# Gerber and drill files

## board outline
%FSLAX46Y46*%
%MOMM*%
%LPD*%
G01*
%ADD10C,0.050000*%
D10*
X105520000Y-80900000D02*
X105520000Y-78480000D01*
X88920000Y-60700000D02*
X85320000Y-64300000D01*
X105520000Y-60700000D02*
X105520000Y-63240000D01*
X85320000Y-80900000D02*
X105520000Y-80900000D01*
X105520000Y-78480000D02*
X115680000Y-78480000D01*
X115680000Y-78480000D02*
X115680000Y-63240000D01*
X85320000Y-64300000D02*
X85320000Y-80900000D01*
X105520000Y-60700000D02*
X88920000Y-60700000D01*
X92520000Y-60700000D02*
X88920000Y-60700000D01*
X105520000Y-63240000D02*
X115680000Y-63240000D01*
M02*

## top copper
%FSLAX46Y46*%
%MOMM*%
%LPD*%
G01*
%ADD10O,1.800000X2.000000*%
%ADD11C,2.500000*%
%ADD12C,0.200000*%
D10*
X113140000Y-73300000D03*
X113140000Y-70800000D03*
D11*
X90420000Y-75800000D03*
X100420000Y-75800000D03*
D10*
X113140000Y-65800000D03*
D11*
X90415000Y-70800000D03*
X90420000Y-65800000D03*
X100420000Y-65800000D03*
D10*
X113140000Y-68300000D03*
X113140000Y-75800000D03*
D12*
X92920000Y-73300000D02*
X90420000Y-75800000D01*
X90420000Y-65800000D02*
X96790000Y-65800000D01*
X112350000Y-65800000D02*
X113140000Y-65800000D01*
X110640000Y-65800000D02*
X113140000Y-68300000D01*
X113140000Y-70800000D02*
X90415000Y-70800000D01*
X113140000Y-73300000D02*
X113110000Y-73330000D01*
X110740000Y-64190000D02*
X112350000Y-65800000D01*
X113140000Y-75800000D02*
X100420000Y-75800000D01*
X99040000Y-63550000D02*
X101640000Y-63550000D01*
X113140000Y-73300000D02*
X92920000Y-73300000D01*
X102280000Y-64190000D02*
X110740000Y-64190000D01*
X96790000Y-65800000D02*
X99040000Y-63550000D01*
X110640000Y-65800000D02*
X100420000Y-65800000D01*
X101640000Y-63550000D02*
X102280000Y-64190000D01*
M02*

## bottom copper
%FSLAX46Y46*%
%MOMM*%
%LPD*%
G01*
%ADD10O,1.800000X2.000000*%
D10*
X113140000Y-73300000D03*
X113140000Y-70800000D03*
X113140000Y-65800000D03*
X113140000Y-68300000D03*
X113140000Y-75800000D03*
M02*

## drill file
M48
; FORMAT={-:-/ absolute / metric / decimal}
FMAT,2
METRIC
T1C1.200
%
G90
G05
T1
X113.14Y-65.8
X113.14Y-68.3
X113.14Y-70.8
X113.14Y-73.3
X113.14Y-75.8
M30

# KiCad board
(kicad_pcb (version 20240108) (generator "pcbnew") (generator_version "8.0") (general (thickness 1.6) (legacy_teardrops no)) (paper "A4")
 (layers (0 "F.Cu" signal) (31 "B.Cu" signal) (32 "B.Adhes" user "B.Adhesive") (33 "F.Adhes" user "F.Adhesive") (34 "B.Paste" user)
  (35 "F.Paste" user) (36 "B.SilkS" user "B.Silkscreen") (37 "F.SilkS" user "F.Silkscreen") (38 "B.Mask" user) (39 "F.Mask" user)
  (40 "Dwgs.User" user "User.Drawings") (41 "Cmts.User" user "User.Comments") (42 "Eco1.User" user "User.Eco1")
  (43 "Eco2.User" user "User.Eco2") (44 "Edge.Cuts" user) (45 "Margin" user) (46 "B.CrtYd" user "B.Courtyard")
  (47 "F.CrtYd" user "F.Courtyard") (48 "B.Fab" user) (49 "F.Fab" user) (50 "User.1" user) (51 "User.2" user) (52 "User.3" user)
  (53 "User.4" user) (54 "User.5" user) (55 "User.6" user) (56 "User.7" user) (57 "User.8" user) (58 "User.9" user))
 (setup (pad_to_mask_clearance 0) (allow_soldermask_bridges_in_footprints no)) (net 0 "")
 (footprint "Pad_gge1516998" (layer "F.Cu") (at 113.14 73.3 180)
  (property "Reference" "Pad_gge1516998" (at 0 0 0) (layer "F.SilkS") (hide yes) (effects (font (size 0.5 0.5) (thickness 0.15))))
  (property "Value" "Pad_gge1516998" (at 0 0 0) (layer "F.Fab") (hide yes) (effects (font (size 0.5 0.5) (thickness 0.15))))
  (pad "2" thru_hole oval (at 0 0 180) (size 1.8 2) (drill 1.2) (layers "*.Cu" "*.Mask") (remove_unused_layers no)
   (solder_mask_margin 0.0508) (thermal_bridge_angle 0)))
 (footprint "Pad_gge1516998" (layer "F.Cu") (at 113.14 70.8 180)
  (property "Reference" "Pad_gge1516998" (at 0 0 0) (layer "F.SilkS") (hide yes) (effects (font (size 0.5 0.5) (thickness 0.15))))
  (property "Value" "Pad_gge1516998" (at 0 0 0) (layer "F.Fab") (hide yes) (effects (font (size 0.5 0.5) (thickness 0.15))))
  (pad "2" thru_hole oval (at 0 0 180) (size 1.8 2) (drill 1.2) (layers "*.Cu" "*.Mask") (remove_unused_layers no)
   (solder_mask_margin 0.0508) (thermal_bridge_angle 0)))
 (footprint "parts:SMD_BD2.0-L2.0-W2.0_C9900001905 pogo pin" (layer "F.Cu") (at 90.42 75.8)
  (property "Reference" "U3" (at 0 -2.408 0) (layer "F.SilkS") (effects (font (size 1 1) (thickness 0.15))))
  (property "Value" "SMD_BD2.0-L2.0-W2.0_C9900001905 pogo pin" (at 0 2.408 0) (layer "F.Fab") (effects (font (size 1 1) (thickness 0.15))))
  (pad "1" smd circle (at 0 0) (size 2.5 2.5) (layers "F.Cu" "F.Paste" "F.Mask") (thermal_bridge_angle 90)))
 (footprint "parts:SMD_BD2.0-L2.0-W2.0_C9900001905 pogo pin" (layer "F.Cu") (at 100.42 75.8)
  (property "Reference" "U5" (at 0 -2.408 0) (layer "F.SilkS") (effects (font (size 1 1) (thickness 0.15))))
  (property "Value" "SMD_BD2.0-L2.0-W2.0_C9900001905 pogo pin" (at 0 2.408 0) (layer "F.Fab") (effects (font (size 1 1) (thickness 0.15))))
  (pad "1" smd circle (at 0 0) (size 2.5 2.5) (layers "F.Cu" "F.Paste" "F.Mask") (thermal_bridge_angle 90)))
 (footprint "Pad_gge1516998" (layer "F.Cu") (at 113.14 65.8 180)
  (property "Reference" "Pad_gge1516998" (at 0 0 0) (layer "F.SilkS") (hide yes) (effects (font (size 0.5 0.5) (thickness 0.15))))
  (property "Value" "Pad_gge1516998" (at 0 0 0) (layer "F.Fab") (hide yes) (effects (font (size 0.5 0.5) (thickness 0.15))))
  (pad "2" thru_hole oval (at 0 0 180) (size 1.8 2) (drill 1.2) (layers "*.Cu" "*.Mask") (remove_unused_layers no)
   (solder_mask_margin 0.0508) (thermal_bridge_angle 0)))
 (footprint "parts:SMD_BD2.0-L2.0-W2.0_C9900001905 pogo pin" (layer "F.Cu") (at 90.415 70.8)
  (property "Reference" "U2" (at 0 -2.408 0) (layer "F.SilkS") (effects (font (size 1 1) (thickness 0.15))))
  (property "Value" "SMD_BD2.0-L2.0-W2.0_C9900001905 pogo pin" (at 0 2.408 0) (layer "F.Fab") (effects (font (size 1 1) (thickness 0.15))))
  (pad "1" smd circle (at 0 0) (size 2.5 2.5) (layers "F.Cu" "F.Paste" "F.Mask") (thermal_bridge_angle 90)))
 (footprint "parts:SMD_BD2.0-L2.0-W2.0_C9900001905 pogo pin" (layer "F.Cu") (at 90.42 65.8)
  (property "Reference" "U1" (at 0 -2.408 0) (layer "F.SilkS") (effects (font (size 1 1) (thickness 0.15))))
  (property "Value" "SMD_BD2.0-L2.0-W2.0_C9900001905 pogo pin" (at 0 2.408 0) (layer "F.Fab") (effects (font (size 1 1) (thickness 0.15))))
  (pad "1" smd circle (at 0 0) (size 2.5 2.5) (layers "F.Cu" "F.Paste" "F.Mask") (thermal_bridge_angle 90)))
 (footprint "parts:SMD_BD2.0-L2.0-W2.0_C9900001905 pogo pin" (layer "F.Cu") (at 100.42 65.8)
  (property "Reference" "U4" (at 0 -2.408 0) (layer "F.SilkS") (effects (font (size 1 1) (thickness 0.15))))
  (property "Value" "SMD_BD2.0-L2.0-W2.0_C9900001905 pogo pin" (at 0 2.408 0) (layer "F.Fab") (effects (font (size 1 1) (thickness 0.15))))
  (pad "1" smd circle (at 0 0) (size 2.5 2.5) (layers "F.Cu" "F.Paste" "F.Mask") (thermal_bridge_angle 90)))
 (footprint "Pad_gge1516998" (layer "F.Cu") (at 113.14 68.3 180)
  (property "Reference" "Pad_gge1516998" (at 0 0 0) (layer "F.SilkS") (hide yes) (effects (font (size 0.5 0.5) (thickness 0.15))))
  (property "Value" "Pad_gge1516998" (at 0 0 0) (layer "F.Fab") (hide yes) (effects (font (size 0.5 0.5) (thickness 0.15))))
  (pad "2" thru_hole oval (at 0 0 180) (size 1.8 2) (drill 1.2) (layers "*.Cu" "*.Mask") (remove_unused_layers no)
   (solder_mask_margin 0.0508) (thermal_bridge_angle 0)))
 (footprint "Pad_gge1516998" (layer "F.Cu") (at 113.14 75.8 180)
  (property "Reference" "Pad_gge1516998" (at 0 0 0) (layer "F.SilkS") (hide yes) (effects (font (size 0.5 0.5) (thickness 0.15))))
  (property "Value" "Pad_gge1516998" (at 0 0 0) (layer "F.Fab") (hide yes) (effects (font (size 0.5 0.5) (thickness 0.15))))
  (pad "2" thru_hole oval (at 0 0 180) (size 1.8 2) (drill 1.2) (layers "*.Cu" "*.Mask") (remove_unused_layers no)
   (solder_mask_margin 0.0508) (thermal_bridge_angle 0)))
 (gr_line (start 105.52 80.9) (end 105.52 78.48) (stroke (width 0.05) (type default)) (layer "Edge.Cuts"))
 (gr_line (start 88.92 60.7) (end 85.32 64.3) (stroke (width 0.05) (type default)) (layer "Edge.Cuts"))
 (gr_line (start 105.52 60.7) (end 105.52 63.24) (stroke (width 0.05) (type default)) (layer "Edge.Cuts"))
 (gr_line (start 85.32 80.9) (end 105.52 80.9) (stroke (width 0.05) (type default)) (layer "Edge.Cuts"))
 (gr_line (start 105.52 78.48) (end 115.68 78.48) (stroke (width 0.05) (type default)) (layer "Edge.Cuts"))
 (gr_line (start 115.68 78.48) (end 115.68 63.24) (stroke (width 0.05) (type default)) (layer "Edge.Cuts"))
 (gr_line (start 85.32 64.3) (end 85.32 80.9) (stroke (width 0.05) (type default)) (layer "Edge.Cuts"))
 (gr_line (start 105.52 60.7) (end 88.92 60.7) (stroke (width 0.05) (type default)) (layer "Edge.Cuts"))
 (gr_line (start 92.52 60.7) (end 88.92 60.7) (stroke (width 0.05) (type default)) (layer "Edge.Cuts"))
 (gr_line (start 105.52 63.24) (end 115.68 63.24) (stroke (width 0.05) (type default)) (layer "Edge.Cuts"))
 (segment (start 92.92 73.3) (end 90.42 75.8) (width 0.2) (layer "F.Cu") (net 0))
 (segment (start 90.42 65.8) (end 96.79 65.8) (width 0.2) (layer "F.Cu") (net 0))
 (segment (start 112.35 65.8) (end 113.14 65.8) (width 0.2) (layer "F.Cu") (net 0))
 (segment (start 110.64 65.8) (end 113.14 68.3) (width 0.2) (layer "F.Cu") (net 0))
 (segment (start 113.14 70.8) (end 90.415 70.8) (width 0.2) (layer "F.Cu") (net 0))
 (segment (start 113.14 73.3) (end 113.11 73.33) (width 0.2) (layer "F.Cu") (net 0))
 (segment (start 110.74 64.19) (end 112.35 65.8) (width 0.2) (layer "F.Cu") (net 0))
 (segment (start 113.14 75.8) (end 100.42 75.8) (width 0.2) (layer "F.Cu") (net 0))
 (segment (start 99.04 63.55) (end 101.64 63.55) (width 0.2) (layer "F.Cu") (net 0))
 (segment (start 113.14 73.3) (end 92.92 73.3) (width 0.2) (layer "F.Cu") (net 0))
 (segment (start 102.28 64.19) (end 110.74 64.19) (width 0.2) (layer "F.Cu") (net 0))
 (segment (start 96.79 65.8) (end 99.04 63.55) (width 0.2) (layer "F.Cu") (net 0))
 (segment (start 110.64 65.8) (end 100.42 65.8) (width 0.2) (layer "F.Cu") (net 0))
 (segment (start 101.64 63.55) (end 102.28 64.19) (width 0.2) (layer "F.Cu") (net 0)))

